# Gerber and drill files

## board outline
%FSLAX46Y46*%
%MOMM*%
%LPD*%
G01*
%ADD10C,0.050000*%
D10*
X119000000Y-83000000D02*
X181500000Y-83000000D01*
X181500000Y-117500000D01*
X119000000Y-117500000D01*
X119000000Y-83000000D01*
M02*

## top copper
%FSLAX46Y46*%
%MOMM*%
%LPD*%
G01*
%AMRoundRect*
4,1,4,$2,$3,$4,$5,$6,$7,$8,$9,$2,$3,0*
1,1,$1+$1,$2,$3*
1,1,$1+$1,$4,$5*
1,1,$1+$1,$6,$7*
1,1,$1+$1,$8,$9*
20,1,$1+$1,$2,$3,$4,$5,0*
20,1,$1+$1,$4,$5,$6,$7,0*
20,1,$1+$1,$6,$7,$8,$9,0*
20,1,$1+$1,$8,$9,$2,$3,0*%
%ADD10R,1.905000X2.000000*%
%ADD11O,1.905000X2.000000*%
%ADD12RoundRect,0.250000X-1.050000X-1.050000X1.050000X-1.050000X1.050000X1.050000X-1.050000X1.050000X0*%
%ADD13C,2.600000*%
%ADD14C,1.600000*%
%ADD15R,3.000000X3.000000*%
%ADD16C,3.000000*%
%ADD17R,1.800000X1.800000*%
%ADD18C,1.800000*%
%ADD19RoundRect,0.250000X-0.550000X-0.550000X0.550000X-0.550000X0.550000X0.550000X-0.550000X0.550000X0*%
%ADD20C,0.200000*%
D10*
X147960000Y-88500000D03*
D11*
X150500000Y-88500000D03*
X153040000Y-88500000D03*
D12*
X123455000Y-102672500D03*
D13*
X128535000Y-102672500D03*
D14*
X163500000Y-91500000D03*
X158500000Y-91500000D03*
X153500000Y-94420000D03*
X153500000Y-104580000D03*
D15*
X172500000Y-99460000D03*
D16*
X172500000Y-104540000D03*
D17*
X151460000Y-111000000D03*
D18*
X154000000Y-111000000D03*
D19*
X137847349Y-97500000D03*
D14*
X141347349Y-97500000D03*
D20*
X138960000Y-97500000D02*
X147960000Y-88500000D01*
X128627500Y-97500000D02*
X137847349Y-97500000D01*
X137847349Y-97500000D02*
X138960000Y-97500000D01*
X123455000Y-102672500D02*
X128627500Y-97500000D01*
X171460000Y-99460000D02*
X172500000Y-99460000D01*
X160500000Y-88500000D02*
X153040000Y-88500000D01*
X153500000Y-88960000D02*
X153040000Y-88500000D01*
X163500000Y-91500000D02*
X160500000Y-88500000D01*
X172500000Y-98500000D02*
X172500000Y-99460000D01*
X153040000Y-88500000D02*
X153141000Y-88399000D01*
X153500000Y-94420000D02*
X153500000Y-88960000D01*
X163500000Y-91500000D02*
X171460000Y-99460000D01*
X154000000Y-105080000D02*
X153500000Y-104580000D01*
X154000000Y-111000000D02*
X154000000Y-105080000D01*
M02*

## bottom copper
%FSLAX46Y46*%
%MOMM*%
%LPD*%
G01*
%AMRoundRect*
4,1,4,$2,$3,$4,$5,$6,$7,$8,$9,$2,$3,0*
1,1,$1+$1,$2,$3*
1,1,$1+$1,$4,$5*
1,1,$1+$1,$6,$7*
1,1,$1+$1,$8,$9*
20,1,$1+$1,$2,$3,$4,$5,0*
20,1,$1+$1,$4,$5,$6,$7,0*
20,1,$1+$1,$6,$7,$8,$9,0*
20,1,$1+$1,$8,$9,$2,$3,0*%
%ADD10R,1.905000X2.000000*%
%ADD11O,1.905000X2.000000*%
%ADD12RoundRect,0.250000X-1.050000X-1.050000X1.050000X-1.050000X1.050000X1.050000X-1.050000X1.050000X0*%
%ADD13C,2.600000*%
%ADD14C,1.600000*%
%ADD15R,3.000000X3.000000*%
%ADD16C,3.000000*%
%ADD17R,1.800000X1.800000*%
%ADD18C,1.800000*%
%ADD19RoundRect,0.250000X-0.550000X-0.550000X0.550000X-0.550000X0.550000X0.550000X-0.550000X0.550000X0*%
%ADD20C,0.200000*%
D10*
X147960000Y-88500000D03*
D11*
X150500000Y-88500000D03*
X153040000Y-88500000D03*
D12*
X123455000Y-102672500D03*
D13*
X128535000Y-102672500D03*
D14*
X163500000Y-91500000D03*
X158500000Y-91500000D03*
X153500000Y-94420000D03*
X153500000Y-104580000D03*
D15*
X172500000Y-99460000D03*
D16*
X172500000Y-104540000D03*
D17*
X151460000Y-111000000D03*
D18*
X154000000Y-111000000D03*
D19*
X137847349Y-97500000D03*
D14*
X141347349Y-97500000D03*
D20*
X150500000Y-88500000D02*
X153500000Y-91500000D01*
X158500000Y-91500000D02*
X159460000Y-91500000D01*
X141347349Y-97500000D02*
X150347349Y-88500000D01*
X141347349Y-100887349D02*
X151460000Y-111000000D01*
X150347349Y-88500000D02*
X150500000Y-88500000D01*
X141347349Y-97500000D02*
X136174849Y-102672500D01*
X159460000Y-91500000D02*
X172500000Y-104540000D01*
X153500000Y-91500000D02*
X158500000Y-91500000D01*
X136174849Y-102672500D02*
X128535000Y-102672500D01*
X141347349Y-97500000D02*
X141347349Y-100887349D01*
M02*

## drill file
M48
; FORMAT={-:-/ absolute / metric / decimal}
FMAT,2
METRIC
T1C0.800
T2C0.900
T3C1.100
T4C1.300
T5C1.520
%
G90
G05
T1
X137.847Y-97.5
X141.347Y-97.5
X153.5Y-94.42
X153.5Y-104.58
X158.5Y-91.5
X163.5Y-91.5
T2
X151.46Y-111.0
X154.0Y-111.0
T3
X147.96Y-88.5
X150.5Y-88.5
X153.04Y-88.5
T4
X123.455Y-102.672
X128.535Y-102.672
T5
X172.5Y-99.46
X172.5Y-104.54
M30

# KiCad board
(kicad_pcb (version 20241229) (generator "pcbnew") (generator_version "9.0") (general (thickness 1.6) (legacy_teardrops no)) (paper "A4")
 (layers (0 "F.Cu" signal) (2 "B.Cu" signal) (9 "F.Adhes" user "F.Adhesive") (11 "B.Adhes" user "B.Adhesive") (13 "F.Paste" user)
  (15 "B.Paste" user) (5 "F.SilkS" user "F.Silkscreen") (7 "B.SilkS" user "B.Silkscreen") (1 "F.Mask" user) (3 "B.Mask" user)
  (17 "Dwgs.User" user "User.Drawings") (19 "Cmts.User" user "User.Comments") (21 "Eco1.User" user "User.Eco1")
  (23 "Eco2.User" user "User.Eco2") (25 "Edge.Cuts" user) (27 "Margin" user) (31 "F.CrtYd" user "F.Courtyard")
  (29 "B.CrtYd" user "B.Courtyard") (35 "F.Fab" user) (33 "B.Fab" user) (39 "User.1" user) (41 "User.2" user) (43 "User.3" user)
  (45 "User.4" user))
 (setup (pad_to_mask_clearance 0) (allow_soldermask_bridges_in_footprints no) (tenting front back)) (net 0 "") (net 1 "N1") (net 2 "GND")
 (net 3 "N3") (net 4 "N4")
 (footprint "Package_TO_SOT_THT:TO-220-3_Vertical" (layer "F.Cu") (at 147.96 88.5)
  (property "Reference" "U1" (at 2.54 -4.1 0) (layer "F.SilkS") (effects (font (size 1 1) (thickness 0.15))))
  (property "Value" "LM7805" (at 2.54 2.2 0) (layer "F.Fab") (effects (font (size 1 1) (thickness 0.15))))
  (pad "1" thru_hole rect (at 0 0) (size 1.905 2) (drill 1.1) (layers "*.Cu" "*.Mask") (remove_unused_layers no) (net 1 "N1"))
  (pad "2" thru_hole oval (at 2.54 0) (size 1.905 2) (drill 1.1) (layers "*.Cu" "*.Mask") (remove_unused_layers no) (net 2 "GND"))
  (pad "3" thru_hole oval (at 5.08 0) (size 1.905 2) (drill 1.1) (layers "*.Cu" "*.Mask") (remove_unused_layers no) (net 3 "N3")))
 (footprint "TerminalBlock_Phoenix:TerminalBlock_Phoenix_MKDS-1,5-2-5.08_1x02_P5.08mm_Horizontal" (layer "F.Cu") (at 123.455 102.6725)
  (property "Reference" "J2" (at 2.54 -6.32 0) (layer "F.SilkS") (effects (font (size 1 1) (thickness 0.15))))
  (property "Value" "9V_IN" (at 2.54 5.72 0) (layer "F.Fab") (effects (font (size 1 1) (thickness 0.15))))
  (pad "1" thru_hole roundrect (at 0 0) (size 2.6 2.6) (drill 1.3) (layers "*.Cu" "*.Mask") (remove_unused_layers no)
   (roundrect_rratio 0.096154) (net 1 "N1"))
  (pad "2" thru_hole circle (at 5.08 0) (size 2.6 2.6) (drill 1.3) (layers "*.Cu" "*.Mask") (remove_unused_layers no) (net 2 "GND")))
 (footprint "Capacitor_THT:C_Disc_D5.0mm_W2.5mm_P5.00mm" (layer "F.Cu") (at 163.5 91.5 180)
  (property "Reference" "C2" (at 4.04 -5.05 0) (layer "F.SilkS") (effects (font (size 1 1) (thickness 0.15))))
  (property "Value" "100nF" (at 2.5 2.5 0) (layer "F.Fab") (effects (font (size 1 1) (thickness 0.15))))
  (pad "1" thru_hole circle (at 0 0 180) (size 1.6 1.6) (drill 0.8) (layers "*.Cu" "*.Mask") (remove_unused_layers no) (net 3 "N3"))
  (pad "2" thru_hole circle (at 5 0 180) (size 1.6 1.6) (drill 0.8) (layers "*.Cu" "*.Mask") (remove_unused_layers no) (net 2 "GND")))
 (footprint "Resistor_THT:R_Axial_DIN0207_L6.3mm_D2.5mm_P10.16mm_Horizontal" (layer "F.Cu") (at 153.5 94.42 -90)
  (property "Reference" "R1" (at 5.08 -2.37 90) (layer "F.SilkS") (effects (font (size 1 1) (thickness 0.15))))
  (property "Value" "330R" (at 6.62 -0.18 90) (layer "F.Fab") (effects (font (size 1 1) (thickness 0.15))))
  (pad "1" thru_hole circle (at 0 0 270) (size 1.6 1.6) (drill 0.8) (layers "*.Cu" "*.Mask") (remove_unused_layers no) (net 3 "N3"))
  (pad "2" thru_hole circle (at 10.16 0 270) (size 1.6 1.6) (drill 0.8) (layers "*.Cu" "*.Mask") (remove_unused_layers no) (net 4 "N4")))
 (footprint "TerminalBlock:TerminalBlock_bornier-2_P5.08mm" (layer "F.Cu") (at 172.5 99.46 -90)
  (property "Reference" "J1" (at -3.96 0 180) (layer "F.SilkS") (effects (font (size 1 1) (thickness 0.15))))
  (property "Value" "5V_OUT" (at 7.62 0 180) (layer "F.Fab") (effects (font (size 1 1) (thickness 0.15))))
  (pad "1" thru_hole rect (at 0 0 270) (size 3 3) (drill 1.52) (layers "*.Cu" "*.Mask") (remove_unused_layers no) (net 3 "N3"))
  (pad "2" thru_hole circle (at 5.08 0 270) (size 3 3) (drill 1.52) (layers "*.Cu" "*.Mask") (remove_unused_layers no) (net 2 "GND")))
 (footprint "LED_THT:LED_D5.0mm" (layer "F.Cu") (at 151.46 111)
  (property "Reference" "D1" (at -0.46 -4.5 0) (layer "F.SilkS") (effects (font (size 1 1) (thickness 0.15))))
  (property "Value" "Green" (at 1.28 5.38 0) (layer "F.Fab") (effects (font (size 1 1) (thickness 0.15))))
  (pad "1" thru_hole rect (at 0 0) (size 1.8 1.8) (drill 0.9) (layers "*.Cu" "*.Mask") (remove_unused_layers no) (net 2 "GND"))
  (pad "2" thru_hole circle (at 2.54 0) (size 1.8 1.8) (drill 0.9) (layers "*.Cu" "*.Mask") (remove_unused_layers no) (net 4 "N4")))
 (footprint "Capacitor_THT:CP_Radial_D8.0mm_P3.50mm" (layer "F.Cu") (at 137.847349 97.5)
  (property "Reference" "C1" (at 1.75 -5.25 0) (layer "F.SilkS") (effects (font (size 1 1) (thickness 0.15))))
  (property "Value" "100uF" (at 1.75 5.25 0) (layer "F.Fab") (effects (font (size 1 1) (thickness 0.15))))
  (pad "1" thru_hole roundrect (at 0 0) (size 1.6 1.6) (drill 0.8) (layers "*.Cu" "*.Mask") (remove_unused_layers no)
   (roundrect_rratio 0.15625) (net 1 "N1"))
  (pad "2" thru_hole circle (at 3.5 0) (size 1.6 1.6) (drill 0.8) (layers "*.Cu" "*.Mask") (remove_unused_layers no) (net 2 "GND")))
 (gr_rect (start 119 83) (end 181.5 117.5) (stroke (width 0.05) (type default)) (fill no) (layer "Edge.Cuts"))
 (segment (start 138.96 97.5) (end 147.96 88.5) (width 0.2) (layer "F.Cu") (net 1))
 (segment (start 128.6275 97.5) (end 137.847349 97.5) (width 0.2) (layer "F.Cu") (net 1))
 (segment (start 137.847349 97.5) (end 138.96 97.5) (width 0.2) (layer "F.Cu") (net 1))
 (segment (start 123.455 102.6725) (end 128.6275 97.5) (width 0.2) (layer "F.Cu") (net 1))
 (segment (start 150.5 88.5) (end 153.5 91.5) (width 0.2) (layer "B.Cu") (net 2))
 (segment (start 158.5 91.5) (end 159.46 91.5) (width 0.2) (layer "B.Cu") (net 2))
 (segment (start 141.347349 97.5) (end 150.347349 88.5) (width 0.2) (layer "B.Cu") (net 2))
 (segment (start 141.347349 100.887349) (end 151.46 111) (width 0.2) (layer "B.Cu") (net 2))
 (segment (start 150.347349 88.5) (end 150.5 88.5) (width 0.2) (layer "B.Cu") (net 2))
 (segment (start 141.347349 97.5) (end 136.174849 102.6725) (width 0.2) (layer "B.Cu") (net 2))
 (segment (start 159.46 91.5) (end 172.5 104.54) (width 0.2) (layer "B.Cu") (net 2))
 (segment (start 153.5 91.5) (end 158.5 91.5) (width 0.2) (layer "B.Cu") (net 2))
 (segment (start 136.174849 102.6725) (end 128.535 102.6725) (width 0.2) (layer "B.Cu") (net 2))
 (segment (start 141.347349 97.5) (end 141.347349 100.887349) (width 0.2) (layer "B.Cu") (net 2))
 (segment (start 171.46 99.46) (end 172.5 99.46) (width 0.2) (layer "F.Cu") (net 3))
 (segment (start 160.5 88.5) (end 153.04 88.5) (width 0.2) (layer "F.Cu") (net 3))
 (segment (start 153.5 88.96) (end 153.04 88.5) (width 0.2) (layer "F.Cu") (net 3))
 (segment (start 163.5 91.5) (end 160.5 88.5) (width 0.2) (layer "F.Cu") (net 3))
 (segment (start 172.5 98.5) (end 172.5 99.46) (width 0.2) (layer "F.Cu") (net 3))
 (segment (start 153.04 88.5) (end 153.141 88.399) (width 0.2) (layer "F.Cu") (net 3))
 (segment (start 153.5 94.42) (end 153.5 88.96) (width 0.2) (layer "F.Cu") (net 3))
 (segment (start 163.5 91.5) (end 171.46 99.46) (width 0.2) (layer "F.Cu") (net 3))
 (segment (start 154 105.08) (end 153.5 104.58) (width 0.2) (layer "F.Cu") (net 4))
 (segment (start 154 111) (end 154 105.08) (width 0.2) (layer "F.Cu") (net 4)))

